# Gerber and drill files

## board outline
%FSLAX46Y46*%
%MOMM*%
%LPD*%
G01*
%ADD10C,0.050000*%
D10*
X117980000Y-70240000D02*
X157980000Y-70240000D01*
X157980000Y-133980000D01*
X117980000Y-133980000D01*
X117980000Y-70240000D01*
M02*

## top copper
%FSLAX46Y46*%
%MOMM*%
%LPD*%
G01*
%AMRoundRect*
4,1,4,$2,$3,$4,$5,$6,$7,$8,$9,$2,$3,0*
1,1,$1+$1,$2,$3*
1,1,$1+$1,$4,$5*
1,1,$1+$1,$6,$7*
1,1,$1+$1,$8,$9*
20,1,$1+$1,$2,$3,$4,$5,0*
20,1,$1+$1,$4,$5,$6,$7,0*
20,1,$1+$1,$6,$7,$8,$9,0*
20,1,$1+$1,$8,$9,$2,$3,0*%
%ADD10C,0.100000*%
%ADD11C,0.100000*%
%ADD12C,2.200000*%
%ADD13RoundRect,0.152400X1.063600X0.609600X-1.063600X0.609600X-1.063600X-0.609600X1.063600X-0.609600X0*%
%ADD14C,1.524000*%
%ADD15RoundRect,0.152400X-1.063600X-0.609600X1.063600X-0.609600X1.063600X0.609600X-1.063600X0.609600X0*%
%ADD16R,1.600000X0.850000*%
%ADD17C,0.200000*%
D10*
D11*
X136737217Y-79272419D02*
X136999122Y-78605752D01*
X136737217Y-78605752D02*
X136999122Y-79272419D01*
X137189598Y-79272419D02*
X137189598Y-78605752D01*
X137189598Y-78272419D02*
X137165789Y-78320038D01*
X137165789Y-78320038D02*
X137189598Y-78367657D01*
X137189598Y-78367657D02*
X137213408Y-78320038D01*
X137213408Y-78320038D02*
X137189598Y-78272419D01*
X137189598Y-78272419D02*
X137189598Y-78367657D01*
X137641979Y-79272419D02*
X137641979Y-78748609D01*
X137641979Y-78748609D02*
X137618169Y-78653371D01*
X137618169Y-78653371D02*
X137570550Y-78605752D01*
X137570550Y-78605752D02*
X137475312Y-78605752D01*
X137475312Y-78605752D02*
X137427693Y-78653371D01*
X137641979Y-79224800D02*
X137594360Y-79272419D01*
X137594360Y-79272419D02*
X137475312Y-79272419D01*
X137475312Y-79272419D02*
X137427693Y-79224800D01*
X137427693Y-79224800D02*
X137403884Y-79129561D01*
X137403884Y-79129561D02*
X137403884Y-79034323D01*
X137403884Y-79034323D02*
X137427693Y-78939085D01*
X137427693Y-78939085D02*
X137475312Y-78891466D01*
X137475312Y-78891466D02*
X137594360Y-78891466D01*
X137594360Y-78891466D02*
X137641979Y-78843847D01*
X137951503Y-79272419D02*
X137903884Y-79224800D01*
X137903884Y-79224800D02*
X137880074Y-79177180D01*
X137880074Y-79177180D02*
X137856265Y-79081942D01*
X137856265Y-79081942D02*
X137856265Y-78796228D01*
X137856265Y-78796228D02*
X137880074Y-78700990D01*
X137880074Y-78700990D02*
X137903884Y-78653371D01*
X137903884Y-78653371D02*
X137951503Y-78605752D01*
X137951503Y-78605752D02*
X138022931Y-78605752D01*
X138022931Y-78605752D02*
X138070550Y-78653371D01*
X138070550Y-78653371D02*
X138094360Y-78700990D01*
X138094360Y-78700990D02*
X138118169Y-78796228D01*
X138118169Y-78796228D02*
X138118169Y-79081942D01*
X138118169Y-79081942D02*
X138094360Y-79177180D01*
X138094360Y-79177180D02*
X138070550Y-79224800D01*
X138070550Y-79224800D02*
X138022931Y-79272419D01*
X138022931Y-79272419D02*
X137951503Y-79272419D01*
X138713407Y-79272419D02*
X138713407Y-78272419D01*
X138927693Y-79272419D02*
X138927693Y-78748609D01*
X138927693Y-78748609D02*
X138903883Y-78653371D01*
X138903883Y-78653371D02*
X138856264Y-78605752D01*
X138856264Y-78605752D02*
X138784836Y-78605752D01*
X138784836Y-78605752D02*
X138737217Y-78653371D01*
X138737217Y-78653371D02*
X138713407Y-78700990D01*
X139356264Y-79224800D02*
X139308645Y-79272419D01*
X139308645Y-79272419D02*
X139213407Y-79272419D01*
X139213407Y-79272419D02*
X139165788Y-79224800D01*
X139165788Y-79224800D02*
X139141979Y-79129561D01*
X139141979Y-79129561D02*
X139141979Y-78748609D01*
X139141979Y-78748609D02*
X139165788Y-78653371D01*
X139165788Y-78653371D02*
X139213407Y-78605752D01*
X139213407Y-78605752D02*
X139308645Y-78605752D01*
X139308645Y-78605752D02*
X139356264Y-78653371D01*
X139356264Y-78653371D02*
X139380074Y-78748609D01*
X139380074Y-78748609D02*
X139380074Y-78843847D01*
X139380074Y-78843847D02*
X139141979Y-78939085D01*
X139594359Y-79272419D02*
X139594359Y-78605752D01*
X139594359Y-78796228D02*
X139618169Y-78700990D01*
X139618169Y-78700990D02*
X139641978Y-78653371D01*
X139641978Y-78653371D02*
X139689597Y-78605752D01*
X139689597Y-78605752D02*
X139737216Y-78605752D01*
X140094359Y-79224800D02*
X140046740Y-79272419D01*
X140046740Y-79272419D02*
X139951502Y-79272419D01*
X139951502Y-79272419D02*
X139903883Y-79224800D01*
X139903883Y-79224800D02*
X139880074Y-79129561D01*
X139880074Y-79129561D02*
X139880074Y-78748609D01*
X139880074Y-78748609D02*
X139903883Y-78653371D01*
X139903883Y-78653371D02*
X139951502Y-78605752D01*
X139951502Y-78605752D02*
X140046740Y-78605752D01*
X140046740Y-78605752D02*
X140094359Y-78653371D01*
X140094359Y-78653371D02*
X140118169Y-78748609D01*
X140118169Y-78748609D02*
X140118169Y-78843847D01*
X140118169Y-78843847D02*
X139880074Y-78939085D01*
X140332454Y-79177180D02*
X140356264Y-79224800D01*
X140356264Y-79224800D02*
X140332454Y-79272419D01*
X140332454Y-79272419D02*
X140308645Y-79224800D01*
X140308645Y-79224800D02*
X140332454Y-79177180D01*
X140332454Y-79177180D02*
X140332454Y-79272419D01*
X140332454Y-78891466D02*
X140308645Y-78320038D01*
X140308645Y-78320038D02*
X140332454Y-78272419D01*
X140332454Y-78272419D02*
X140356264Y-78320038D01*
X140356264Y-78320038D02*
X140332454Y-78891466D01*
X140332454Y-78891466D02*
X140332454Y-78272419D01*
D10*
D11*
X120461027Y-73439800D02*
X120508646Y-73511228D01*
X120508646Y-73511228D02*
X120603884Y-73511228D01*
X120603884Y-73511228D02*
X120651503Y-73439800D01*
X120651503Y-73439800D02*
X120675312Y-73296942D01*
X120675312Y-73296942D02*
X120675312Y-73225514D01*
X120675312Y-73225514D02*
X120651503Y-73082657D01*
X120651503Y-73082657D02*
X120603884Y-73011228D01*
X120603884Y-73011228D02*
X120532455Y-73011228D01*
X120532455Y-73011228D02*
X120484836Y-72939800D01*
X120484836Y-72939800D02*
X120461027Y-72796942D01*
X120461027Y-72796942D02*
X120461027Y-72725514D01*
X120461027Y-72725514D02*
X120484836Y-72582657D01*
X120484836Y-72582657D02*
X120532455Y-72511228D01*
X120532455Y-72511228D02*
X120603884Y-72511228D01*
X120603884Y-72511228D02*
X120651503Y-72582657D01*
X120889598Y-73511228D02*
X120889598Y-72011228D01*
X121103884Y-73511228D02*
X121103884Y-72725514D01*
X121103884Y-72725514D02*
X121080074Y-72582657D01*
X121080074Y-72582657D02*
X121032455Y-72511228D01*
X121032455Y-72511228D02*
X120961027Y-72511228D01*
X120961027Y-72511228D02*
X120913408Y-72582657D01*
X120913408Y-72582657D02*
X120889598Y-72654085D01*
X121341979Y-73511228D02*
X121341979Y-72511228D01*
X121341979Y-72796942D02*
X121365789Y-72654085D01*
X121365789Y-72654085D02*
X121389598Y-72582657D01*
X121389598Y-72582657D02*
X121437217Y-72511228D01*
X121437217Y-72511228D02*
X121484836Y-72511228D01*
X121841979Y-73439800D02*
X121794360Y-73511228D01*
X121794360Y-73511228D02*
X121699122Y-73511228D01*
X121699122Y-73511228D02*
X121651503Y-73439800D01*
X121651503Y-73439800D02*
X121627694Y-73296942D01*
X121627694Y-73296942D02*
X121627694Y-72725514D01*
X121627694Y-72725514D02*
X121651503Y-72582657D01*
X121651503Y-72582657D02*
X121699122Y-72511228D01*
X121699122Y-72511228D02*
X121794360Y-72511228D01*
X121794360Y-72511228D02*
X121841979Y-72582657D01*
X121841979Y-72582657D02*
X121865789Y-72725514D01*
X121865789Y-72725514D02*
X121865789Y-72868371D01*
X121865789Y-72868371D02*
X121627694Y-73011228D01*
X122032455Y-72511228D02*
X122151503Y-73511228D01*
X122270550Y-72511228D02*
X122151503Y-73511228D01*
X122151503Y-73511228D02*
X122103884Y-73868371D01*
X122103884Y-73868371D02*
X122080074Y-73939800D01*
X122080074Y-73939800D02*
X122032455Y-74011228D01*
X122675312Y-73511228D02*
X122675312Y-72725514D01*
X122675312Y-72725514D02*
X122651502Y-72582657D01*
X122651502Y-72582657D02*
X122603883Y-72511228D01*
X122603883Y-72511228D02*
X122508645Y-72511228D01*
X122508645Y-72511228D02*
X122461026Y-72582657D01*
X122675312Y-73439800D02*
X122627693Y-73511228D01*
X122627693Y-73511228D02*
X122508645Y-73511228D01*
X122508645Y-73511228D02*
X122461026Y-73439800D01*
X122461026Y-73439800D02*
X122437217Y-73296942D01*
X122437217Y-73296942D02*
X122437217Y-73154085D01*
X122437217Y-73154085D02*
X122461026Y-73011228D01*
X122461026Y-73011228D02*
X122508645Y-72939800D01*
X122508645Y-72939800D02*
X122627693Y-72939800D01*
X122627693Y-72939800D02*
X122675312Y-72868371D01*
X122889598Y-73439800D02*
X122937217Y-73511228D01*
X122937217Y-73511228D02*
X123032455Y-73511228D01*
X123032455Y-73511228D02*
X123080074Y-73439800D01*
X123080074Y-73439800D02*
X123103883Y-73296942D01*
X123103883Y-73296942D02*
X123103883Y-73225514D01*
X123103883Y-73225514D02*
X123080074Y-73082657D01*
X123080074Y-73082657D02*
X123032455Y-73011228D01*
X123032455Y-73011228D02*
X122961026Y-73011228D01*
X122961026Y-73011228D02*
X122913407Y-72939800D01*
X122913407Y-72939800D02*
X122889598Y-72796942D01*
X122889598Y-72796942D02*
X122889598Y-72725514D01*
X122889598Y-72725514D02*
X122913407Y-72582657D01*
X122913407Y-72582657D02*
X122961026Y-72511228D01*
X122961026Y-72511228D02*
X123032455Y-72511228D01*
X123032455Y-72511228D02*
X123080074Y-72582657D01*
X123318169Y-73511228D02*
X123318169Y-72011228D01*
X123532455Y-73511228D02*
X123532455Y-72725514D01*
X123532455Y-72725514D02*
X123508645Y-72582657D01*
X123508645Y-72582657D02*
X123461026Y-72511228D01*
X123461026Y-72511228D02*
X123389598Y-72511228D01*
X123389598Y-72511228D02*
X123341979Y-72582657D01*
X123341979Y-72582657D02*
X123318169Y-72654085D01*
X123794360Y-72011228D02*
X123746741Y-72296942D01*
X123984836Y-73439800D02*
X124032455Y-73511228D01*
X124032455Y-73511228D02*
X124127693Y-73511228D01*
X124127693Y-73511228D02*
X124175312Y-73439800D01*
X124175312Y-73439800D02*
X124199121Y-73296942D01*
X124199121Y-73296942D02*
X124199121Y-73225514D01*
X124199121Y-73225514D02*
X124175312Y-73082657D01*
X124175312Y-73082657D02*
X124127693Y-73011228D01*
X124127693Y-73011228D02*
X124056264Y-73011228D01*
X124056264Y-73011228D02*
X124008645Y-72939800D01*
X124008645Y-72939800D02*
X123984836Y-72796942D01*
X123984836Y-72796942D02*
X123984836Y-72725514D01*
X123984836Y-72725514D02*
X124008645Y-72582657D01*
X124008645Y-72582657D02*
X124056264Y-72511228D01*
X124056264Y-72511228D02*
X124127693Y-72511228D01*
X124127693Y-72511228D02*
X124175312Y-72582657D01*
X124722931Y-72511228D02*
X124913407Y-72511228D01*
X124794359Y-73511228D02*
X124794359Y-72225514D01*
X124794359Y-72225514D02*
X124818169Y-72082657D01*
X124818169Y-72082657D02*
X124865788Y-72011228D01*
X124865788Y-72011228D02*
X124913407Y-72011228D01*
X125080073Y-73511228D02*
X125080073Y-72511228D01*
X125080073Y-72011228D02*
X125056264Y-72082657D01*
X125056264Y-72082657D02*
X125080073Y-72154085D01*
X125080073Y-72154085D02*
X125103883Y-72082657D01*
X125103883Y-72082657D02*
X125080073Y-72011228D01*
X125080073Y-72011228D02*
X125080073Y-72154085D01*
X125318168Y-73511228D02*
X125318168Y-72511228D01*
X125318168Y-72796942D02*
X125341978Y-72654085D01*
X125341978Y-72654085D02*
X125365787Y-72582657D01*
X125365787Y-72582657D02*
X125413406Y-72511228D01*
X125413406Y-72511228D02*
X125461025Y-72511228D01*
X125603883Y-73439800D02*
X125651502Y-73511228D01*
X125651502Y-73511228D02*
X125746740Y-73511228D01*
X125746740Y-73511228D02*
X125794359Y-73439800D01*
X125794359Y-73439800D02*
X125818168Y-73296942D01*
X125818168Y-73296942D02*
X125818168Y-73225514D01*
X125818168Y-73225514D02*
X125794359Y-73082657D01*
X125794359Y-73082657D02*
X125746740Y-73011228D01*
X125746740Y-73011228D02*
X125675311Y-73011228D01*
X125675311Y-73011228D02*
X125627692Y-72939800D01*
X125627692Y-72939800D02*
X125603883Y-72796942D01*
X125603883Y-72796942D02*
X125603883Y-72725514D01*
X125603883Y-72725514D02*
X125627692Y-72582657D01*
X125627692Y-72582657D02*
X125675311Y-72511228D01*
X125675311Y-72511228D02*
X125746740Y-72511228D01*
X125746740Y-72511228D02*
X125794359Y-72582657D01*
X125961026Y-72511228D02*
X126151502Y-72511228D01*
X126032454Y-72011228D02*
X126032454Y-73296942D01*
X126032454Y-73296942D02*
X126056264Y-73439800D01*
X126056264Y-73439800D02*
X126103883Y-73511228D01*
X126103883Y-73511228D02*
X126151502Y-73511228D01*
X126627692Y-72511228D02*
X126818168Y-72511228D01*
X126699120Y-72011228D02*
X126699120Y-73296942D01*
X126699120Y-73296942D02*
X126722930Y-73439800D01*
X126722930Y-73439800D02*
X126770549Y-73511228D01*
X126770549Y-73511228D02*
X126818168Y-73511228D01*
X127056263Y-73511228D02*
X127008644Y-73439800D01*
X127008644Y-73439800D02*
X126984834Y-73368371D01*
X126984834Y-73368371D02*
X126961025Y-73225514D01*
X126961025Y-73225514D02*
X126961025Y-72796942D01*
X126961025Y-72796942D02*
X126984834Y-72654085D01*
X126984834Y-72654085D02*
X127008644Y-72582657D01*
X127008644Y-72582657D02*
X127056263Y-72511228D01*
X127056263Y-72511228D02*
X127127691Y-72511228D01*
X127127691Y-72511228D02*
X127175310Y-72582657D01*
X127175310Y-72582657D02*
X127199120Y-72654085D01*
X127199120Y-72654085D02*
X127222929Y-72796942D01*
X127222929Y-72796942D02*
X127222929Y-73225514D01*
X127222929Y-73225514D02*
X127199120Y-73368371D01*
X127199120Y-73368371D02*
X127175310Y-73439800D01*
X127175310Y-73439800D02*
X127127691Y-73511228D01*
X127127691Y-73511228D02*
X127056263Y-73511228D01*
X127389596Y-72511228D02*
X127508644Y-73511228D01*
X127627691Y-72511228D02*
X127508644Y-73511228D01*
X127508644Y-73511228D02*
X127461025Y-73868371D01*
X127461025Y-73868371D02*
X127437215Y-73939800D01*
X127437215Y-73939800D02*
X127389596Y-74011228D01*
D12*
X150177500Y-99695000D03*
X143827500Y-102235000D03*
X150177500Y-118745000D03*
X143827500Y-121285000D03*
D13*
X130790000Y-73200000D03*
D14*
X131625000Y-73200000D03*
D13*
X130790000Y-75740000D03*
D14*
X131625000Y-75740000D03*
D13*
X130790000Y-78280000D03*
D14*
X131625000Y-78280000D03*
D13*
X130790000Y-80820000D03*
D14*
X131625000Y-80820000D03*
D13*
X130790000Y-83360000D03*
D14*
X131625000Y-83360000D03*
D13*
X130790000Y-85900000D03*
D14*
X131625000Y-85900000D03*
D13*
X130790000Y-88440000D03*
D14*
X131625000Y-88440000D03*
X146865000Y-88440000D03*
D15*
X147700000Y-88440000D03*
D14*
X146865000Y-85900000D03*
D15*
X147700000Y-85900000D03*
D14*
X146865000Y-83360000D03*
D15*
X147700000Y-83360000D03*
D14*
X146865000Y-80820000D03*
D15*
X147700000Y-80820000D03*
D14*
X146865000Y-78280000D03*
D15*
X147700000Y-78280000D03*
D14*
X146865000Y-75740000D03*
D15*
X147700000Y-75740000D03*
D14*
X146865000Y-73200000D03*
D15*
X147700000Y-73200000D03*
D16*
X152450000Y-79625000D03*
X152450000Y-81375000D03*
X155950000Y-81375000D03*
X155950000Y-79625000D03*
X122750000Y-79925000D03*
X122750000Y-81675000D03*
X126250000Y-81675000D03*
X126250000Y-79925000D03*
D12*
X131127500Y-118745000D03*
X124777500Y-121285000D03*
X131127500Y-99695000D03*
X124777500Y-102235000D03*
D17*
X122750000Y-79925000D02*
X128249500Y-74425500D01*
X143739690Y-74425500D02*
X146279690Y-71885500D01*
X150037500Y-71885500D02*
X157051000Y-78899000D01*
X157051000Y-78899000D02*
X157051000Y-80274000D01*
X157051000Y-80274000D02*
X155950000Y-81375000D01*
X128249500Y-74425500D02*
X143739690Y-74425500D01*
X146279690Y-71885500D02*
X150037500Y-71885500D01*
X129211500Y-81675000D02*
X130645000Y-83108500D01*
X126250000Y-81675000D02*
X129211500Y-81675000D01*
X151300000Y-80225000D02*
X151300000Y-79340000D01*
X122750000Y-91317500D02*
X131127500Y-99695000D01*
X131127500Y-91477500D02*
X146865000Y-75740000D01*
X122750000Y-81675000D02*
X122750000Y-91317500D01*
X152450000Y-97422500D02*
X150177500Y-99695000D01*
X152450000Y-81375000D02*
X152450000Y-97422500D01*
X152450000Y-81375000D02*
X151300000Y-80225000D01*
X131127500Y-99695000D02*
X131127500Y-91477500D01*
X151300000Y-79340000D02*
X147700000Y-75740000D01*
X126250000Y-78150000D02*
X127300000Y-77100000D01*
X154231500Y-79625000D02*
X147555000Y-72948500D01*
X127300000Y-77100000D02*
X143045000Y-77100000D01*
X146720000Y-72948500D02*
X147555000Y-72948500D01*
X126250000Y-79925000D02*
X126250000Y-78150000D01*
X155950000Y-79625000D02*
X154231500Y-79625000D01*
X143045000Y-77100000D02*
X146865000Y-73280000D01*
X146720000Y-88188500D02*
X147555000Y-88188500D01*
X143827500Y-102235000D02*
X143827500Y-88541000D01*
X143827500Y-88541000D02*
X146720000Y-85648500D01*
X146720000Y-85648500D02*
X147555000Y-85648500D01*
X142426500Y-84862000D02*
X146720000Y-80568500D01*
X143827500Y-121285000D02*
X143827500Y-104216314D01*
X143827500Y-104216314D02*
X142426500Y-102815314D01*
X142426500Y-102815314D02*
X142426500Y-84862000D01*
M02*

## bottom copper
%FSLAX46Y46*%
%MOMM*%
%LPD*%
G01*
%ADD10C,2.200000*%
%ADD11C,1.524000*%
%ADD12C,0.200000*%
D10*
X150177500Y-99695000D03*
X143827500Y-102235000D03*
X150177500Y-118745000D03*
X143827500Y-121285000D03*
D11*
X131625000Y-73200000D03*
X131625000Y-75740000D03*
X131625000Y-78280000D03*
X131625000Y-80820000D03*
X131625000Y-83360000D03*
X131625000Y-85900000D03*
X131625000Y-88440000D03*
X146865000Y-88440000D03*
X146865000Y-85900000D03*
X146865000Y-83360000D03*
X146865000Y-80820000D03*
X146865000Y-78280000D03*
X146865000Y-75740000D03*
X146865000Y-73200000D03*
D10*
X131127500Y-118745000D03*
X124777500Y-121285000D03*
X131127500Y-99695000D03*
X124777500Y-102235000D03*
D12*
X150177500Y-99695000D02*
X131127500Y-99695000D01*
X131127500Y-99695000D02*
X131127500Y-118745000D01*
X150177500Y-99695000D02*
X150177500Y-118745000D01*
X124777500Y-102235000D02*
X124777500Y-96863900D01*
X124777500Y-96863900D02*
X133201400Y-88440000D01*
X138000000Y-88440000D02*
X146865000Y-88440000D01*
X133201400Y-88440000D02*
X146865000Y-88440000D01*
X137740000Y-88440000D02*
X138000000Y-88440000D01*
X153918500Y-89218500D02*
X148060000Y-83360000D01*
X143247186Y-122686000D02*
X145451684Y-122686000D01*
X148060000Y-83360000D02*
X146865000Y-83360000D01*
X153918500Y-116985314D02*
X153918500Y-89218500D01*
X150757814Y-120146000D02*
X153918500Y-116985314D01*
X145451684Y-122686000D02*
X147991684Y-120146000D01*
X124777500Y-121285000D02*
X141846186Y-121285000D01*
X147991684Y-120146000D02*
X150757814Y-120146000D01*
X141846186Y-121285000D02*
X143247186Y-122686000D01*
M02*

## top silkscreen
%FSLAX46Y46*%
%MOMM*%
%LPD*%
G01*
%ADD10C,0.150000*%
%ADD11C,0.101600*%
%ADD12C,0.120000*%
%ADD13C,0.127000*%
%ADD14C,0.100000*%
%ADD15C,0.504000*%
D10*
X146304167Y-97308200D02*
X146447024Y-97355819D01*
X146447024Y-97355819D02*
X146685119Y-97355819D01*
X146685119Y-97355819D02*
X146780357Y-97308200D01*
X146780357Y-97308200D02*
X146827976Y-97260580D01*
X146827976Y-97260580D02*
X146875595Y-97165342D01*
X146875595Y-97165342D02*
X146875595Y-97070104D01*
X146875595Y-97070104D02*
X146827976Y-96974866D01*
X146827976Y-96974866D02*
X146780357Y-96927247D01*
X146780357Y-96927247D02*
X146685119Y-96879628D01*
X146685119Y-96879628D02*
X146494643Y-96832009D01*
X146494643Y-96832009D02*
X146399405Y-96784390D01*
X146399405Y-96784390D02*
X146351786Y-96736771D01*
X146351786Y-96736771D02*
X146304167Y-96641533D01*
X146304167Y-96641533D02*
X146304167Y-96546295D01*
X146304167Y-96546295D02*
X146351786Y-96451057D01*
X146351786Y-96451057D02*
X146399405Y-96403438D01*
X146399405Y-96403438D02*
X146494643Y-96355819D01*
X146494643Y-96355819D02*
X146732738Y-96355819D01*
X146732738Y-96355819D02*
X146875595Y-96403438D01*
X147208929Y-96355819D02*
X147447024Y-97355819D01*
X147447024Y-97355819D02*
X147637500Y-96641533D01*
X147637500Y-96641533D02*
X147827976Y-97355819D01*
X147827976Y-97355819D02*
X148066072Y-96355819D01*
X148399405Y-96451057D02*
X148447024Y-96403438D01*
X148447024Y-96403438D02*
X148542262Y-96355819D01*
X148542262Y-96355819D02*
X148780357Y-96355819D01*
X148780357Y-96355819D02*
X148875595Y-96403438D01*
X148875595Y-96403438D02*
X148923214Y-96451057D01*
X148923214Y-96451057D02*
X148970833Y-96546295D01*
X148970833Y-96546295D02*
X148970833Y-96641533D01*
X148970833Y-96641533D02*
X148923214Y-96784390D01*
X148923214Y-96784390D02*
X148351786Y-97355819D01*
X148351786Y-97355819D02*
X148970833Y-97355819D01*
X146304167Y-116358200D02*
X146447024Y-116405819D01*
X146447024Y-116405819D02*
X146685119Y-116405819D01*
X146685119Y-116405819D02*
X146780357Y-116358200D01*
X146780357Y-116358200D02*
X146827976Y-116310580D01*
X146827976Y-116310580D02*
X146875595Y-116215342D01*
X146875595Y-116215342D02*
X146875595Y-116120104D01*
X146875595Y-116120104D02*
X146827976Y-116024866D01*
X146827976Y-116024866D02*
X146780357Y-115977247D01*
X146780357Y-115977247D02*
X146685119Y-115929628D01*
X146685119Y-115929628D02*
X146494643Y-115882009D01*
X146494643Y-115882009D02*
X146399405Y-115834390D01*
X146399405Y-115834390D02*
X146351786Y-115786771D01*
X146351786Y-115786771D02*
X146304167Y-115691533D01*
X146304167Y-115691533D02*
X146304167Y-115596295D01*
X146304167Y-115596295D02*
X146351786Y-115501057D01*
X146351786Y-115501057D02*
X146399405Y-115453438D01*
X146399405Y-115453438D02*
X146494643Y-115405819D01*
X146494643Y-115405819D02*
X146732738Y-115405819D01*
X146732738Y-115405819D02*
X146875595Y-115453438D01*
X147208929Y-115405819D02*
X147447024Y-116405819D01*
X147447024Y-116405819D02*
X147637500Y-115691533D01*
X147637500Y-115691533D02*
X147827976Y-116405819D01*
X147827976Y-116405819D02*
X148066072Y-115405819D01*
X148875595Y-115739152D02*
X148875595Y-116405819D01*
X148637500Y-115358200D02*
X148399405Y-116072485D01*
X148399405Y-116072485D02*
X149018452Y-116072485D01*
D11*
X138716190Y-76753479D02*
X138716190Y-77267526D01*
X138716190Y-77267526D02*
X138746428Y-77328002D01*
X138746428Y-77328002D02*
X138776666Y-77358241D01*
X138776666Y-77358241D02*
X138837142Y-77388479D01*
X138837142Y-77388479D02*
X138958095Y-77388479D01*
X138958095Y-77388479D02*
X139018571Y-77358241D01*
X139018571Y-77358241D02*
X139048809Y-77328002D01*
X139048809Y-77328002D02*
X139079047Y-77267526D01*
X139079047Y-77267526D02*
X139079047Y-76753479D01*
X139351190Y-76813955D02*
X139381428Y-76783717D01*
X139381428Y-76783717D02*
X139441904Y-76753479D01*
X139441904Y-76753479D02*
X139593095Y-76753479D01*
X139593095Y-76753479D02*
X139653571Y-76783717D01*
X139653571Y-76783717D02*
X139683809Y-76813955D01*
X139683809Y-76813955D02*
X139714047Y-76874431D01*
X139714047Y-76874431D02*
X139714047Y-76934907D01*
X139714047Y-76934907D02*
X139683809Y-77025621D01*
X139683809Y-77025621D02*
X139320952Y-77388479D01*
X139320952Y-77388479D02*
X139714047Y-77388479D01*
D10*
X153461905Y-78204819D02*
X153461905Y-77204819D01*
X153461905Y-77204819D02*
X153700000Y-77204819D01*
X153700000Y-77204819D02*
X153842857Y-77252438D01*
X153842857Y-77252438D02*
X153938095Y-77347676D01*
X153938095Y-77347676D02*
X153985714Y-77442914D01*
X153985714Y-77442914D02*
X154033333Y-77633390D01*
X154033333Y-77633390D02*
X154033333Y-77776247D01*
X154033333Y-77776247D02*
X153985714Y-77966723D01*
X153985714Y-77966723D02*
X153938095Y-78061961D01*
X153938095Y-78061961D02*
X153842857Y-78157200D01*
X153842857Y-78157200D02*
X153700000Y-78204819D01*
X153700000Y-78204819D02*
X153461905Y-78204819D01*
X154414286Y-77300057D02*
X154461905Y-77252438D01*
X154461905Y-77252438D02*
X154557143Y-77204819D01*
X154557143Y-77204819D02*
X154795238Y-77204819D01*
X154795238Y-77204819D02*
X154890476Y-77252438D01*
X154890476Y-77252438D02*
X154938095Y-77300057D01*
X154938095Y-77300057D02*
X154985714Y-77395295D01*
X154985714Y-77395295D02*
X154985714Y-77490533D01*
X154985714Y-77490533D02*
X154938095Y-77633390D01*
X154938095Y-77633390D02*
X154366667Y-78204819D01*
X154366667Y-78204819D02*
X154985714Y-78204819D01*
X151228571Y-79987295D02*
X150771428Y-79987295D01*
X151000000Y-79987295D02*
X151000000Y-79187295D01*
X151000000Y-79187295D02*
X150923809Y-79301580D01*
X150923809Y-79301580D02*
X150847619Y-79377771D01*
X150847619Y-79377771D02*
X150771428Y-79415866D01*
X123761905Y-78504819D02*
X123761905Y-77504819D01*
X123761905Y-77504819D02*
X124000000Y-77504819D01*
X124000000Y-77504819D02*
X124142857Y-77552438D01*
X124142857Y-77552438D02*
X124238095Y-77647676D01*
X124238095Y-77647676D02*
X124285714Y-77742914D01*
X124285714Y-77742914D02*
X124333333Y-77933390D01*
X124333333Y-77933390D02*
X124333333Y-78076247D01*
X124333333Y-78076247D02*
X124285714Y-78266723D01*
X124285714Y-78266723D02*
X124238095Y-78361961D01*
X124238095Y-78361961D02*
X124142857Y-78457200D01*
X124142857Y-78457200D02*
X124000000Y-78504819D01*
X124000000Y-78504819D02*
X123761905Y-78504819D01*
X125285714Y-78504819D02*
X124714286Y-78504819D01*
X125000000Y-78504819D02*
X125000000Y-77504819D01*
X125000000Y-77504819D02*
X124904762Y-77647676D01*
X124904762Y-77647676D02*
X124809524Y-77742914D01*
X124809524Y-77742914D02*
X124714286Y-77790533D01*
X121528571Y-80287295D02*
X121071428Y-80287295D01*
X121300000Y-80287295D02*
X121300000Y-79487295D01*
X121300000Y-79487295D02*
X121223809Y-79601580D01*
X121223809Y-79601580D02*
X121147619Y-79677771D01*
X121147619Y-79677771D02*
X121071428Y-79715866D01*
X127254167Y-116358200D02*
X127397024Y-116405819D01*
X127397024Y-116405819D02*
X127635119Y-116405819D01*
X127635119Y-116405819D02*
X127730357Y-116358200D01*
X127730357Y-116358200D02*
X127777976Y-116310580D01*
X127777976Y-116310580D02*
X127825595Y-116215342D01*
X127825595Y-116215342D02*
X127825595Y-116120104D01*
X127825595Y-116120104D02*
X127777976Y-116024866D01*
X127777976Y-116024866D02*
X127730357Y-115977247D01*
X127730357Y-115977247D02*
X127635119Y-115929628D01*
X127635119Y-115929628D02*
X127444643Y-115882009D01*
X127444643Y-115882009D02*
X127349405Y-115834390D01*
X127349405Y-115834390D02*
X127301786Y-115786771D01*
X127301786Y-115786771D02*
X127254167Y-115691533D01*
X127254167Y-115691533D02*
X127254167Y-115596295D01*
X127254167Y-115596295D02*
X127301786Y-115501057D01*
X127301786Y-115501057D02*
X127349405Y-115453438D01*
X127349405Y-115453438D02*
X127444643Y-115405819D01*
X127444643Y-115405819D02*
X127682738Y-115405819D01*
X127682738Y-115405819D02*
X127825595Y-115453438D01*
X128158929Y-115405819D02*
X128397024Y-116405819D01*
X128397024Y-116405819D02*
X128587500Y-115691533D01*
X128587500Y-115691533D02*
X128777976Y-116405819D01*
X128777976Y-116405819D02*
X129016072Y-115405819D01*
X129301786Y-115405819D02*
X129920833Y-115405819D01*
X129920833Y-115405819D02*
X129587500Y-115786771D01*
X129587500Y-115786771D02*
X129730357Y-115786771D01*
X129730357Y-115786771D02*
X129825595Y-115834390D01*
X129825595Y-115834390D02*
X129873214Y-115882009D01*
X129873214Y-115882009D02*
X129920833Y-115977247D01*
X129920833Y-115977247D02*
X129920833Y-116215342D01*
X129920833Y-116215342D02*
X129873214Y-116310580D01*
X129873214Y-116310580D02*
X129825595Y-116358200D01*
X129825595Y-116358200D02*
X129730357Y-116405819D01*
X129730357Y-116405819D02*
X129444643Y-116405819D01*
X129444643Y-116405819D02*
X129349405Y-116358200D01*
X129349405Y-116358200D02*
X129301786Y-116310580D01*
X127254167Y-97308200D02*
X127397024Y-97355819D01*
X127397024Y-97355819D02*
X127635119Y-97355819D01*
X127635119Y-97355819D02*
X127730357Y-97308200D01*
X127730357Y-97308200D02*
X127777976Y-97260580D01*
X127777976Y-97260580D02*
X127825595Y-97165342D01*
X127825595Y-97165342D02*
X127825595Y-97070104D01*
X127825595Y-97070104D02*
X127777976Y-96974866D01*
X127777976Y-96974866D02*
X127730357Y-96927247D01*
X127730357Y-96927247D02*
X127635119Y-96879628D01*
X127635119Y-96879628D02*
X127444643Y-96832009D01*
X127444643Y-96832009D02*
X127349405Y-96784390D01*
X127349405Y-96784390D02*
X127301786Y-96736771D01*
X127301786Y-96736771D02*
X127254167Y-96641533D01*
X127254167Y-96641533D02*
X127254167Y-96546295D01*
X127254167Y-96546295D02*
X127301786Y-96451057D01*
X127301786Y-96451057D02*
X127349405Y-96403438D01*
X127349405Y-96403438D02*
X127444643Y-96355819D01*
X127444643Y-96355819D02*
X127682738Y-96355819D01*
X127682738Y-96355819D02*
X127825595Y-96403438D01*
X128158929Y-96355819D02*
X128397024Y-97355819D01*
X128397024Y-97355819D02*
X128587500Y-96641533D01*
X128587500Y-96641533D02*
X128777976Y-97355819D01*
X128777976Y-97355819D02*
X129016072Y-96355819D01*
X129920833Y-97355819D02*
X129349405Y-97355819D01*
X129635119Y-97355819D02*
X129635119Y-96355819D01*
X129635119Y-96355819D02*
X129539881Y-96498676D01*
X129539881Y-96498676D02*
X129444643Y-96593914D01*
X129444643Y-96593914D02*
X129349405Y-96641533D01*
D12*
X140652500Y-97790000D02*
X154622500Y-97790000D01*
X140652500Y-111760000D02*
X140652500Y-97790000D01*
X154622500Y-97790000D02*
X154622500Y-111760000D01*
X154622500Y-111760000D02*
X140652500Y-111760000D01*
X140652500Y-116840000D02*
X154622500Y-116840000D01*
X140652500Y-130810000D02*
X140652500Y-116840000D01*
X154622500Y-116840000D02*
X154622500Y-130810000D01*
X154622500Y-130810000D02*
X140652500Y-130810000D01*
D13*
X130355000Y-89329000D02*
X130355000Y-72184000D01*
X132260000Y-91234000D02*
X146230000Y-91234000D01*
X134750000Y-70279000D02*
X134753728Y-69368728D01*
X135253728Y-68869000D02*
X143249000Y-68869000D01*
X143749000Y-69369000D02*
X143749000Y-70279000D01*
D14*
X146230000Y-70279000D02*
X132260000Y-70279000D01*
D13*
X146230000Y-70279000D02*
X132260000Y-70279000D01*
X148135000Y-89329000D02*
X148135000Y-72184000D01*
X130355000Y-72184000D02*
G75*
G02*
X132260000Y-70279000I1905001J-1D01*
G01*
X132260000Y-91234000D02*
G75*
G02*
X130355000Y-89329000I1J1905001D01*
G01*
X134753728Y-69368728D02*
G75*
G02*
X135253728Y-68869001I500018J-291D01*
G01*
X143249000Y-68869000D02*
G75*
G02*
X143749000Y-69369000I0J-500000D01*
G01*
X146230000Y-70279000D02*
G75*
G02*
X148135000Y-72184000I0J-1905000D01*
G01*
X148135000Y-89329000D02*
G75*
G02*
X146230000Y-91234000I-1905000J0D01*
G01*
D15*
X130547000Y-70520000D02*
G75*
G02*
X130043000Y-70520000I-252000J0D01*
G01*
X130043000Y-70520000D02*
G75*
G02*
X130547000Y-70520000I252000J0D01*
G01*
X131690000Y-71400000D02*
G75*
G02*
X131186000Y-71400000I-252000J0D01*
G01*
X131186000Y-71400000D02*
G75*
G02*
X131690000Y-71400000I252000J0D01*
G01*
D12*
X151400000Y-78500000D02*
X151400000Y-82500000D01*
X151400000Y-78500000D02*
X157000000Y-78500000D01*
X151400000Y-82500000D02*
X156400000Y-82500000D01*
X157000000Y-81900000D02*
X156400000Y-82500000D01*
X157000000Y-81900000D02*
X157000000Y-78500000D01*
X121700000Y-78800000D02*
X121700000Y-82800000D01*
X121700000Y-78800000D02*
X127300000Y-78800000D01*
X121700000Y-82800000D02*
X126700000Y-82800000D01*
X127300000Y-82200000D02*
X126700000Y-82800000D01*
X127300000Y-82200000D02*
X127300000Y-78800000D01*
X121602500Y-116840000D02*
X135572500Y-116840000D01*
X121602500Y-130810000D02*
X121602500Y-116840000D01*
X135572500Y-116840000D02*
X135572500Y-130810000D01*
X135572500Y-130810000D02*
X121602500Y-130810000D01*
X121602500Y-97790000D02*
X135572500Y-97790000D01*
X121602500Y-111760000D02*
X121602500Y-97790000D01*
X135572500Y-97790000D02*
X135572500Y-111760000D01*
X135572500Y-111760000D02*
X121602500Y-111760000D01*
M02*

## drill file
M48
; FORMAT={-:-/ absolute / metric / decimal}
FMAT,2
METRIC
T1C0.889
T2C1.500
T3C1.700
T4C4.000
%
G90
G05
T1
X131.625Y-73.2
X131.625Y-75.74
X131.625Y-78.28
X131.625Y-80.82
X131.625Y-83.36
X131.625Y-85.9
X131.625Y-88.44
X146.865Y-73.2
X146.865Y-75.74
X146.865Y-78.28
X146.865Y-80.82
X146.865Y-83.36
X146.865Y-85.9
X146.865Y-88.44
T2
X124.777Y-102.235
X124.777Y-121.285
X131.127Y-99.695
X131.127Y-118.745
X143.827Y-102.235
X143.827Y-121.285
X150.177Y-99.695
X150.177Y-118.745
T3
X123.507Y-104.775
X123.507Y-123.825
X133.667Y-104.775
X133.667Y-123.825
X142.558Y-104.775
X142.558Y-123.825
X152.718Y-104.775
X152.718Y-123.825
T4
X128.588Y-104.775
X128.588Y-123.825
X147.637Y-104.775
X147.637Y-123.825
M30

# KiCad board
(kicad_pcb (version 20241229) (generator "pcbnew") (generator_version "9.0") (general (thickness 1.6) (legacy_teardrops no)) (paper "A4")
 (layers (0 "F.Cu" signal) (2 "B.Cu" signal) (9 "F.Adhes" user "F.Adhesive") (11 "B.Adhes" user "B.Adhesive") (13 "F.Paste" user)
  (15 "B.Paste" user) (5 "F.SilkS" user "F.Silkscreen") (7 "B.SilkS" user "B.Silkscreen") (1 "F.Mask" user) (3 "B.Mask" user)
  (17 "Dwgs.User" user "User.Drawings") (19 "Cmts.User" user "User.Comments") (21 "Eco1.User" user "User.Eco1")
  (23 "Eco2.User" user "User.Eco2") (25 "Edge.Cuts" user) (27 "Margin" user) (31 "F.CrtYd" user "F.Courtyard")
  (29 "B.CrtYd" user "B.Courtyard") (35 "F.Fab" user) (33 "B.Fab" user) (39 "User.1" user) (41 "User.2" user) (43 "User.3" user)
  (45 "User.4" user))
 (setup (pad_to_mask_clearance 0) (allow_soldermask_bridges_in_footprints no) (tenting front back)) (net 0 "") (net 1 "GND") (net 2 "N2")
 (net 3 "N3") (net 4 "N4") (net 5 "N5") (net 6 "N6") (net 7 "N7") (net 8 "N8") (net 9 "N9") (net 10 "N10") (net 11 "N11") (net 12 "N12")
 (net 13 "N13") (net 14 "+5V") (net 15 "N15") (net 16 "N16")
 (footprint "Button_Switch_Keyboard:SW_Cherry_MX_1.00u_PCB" (layer "F.Cu") (at 150.1775 99.695)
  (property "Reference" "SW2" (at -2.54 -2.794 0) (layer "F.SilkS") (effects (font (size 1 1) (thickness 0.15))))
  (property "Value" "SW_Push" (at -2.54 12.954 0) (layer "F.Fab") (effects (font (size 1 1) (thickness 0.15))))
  (fp_line (start -9.525 -1.905) (end 4.445 -1.905) (stroke (width 0.12) (type solid)) (layer "F.SilkS"))
  (fp_line (start -9.525 12.065) (end -9.525 -1.905) (stroke (width 0.12) (type solid)) (layer "F.SilkS"))
  (fp_line (start 4.445 -1.905) (end 4.445 12.065) (stroke (width 0.12) (type solid)) (layer "F.SilkS"))
  (fp_line (start 4.445 12.065) (end -9.525 12.065) (stroke (width 0.12) (type solid)) (layer "F.SilkS"))
  (pad "" np_thru_hole circle (at -7.62 5.08) (size 1.7 1.7) (drill 1.7) (layers "*.Cu" "*.Mask"))
  (pad "" np_thru_hole circle (at -2.54 5.08) (size 4 4) (drill 4) (layers "*.Cu" "*.Mask"))
  (pad "" np_thru_hole circle (at 2.54 5.08) (size 1.7 1.7) (drill 1.7) (layers "*.Cu" "*.Mask"))
  (pad "1" thru_hole circle (at 0 0) (size 2.2 2.2) (drill 1.5) (layers "*.Cu" "*.Mask") (remove_unused_layers no) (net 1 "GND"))
  (pad "2" thru_hole circle (at -6.35 2.54) (size 2.2 2.2) (drill 1.5) (layers "*.Cu" "*.Mask") (remove_unused_layers no) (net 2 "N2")))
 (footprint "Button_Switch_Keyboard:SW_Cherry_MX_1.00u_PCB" (layer "F.Cu") (at 150.1775 118.745)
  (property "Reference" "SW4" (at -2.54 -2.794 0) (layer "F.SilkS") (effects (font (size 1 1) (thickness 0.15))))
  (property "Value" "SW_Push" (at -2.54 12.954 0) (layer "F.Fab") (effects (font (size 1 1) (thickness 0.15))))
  (fp_line (start -9.525 -1.905) (end 4.445 -1.905) (stroke (width 0.12) (type solid)) (layer "F.SilkS"))
  (fp_line (start -9.525 12.065) (end -9.525 -1.905) (stroke (width 0.12) (type solid)) (layer "F.SilkS"))
  (fp_line (start 4.445 -1.905) (end 4.445 12.065) (stroke (width 0.12) (type solid)) (layer "F.SilkS"))
  (fp_line (start 4.445 12.065) (end -9.525 12.065) (stroke (width 0.12) (type solid)) (layer "F.SilkS"))
  (pad "" np_thru_hole circle (at -7.62 5.08) (size 1.7 1.7) (drill 1.7) (layers "*.Cu" "*.Mask"))
  (pad "" np_thru_hole circle (at -2.54 5.08) (size 4 4) (drill 4) (layers "*.Cu" "*.Mask"))
  (pad "" np_thru_hole circle (at 2.54 5.08) (size 1.7 1.7) (drill 1.7) (layers "*.Cu" "*.Mask"))
  (pad "1" thru_hole circle (at 0 0) (size 2.2 2.2) (drill 1.5) (layers "*.Cu" "*.Mask") (remove_unused_layers no) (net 1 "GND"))
  (pad "2" thru_hole circle (at -6.35 2.54) (size 2.2 2.2) (drill 1.5) (layers "*.Cu" "*.Mask") (remove_unused_layers no) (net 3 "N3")))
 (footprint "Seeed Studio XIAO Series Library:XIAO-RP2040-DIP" (layer "F.Cu") (at 139.245 80.82)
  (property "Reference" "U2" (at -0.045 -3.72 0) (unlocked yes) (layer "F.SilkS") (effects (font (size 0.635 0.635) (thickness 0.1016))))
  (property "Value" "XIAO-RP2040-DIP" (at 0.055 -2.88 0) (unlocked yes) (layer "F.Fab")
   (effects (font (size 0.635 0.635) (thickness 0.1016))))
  (fp_line (start -8.89 8.509) (end -8.89 -8.636) (stroke (width 0.127) (type solid)) (layer "F.SilkS"))
  (fp_line (start -6.985 10.414) (end 6.985 10.414) (stroke (width 0.127) (type solid)) (layer "F.SilkS"))
  (fp_line (start -4.495 -10.541) (end -4.491272 -11.451272) (stroke (width 0.127) (type solid)) (layer "F.SilkS"))
  (fp_line (start -3.991272 -11.951) (end 4.004 -11.951) (stroke (width 0.127) (type solid)) (layer "F.SilkS"))
  (fp_line (start 4.504 -11.451) (end 4.504 -10.541) (stroke (width 0.127) (type solid)) (layer "F.SilkS"))
  (fp_line (start 6.985 -10.541) (end -6.985 -10.541) (stroke (width 0.1) (type solid)) (layer "F.SilkS"))
  (fp_line (start 6.985 -10.541) (end -6.985 -10.541) (stroke (width 0.127) (type solid)) (layer "F.SilkS"))
  (fp_line (start 8.89 8.509) (end 8.89 -8.636) (stroke (width 0.127) (type solid)) (layer "F.SilkS"))
  (fp_arc (start -8.89 -8.636) (mid -8.332038 -9.983038) (end -6.985 -10.541) (stroke (width 0.127) (type solid)) (layer "F.SilkS"))
  (fp_arc (start -6.985 10.414) (mid -8.332038 9.856038) (end -8.89 8.509) (stroke (width 0.127) (type solid)) (layer "F.SilkS"))
  (fp_arc (start -4.491272 -11.451272) (mid -4.344728 -11.80464) (end -3.991272 -11.951) (stroke (width 0.127) (type default))
   (layer "F.SilkS"))
  (fp_arc (start 4.004 -11.951) (mid 4.357553 -11.804553) (end 4.504 -11.451) (stroke (width 0.127) (type default)) (layer "F.SilkS"))
  (fp_arc (start 6.985 -10.541) (mid 8.332038 -9.983038) (end 8.89 -8.636) (stroke (width 0.127) (type solid)) (layer "F.SilkS"))
  (fp_arc (start 8.89 8.509) (mid 8.332038 9.856038) (end 6.985 10.414) (stroke (width 0.127) (type solid)) (layer "F.SilkS"))
  (fp_circle (center -8.95 -10.3) (end -8.95 -10.554) (stroke (width 0.5) (type solid)) (fill yes) (layer "F.SilkS"))
  (fp_circle (center -7.807 -9.42) (end -7.807 -9.674) (stroke (width 0.5) (type solid)) (fill yes) (layer "F.SilkS"))
  (pad "1" smd roundrect (at -8.455 -7.62 180) (size 2.432 1.524) (layers "F.Cu" "F.Mask") (roundrect_rratio 0.1) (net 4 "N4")
   (thermal_bridge_angle 45))
  (pad "1" thru_hole circle (at -7.62 -7.62 180) (size 1.524 1.524) (drill 0.889) (layers "*.Cu" "*.Mask") (remove_unused_layers no)
   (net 4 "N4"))
  (pad "2" smd roundrect (at -8.455 -5.08 180) (size 2.432 1.524) (layers "F.Cu" "F.Mask") (roundrect_rratio 0.1) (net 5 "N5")
   (thermal_bridge_angle 45))
  (pad "2" thru_hole circle (at -7.62 -5.08 180) (size 1.524 1.524) (drill 0.889) (layers "*.Cu" "*.Mask") (remove_unused_layers no)
   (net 5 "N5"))
  (pad "3" smd roundrect (at -8.455 -2.54 180) (size 2.432 1.524) (layers "F.Cu" "F.Mask") (roundrect_rratio 0.1) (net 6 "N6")
   (thermal_bridge_angle 45))
  (pad "3" thru_hole circle (at -7.62 -2.54 180) (size 1.524 1.524) (drill 0.889) (layers "*.Cu" "*.Mask") (remove_unused_layers no)
   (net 6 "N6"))
  (pad "4" smd roundrect (at -8.455 0 180) (size 2.432 1.524) (layers "F.Cu" "F.Mask") (roundrect_rratio 0.1) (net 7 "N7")
   (thermal_bridge_angle 45))
  (pad "4" thru_hole circle (at -7.62 0 180) (size 1.524 1.524) (drill 0.889) (layers "*.Cu" "*.Mask") (remove_unused_layers no)
   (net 7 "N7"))
  (pad "5" smd roundrect (at -8.455 2.54 180) (size 2.432 1.524) (layers "F.Cu" "F.Mask") (roundrect_rratio 0.1) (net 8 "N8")
   (thermal_bridge_angle 45))
  (pad "5" thru_hole circle (at -7.62 2.54 180) (size 1.524 1.524) (drill 0.889) (layers "*.Cu" "*.Mask") (remove_unused_layers no)
   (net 8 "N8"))
  (pad "6" smd roundrect (at -8.455 5.08 180) (size 2.432 1.524) (layers "F.Cu" "F.Mask") (roundrect_rratio 0.1) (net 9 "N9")
   (thermal_bridge_angle 45))
  (pad "6" thru_hole circle (at -7.62 5.08 180) (size 1.524 1.524) (drill 0.889) (layers "*.Cu" "*.Mask") (remove_unused_layers no)
   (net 9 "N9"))
  (pad "7" smd roundrect (at -8.455 7.62 180) (size 2.432 1.524) (layers "F.Cu" "F.Mask") (roundrect_rratio 0.1) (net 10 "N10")
   (thermal_bridge_angle 45))
  (pad "7" thru_hole circle (at -7.62 7.62 180) (size 1.524 1.524) (drill 0.889) (layers "*.Cu" "*.Mask") (remove_unused_layers no)
   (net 10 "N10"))
  (pad "8" thru_hole circle (at 7.62 7.62) (size 1.524 1.524) (drill 0.889) (layers "*.Cu" "*.Mask") (remove_unused_layers no)
   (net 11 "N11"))
  (pad "8" smd roundrect (at 8.455 7.62) (size 2.432 1.524) (layers "F.Cu" "F.Mask") (roundrect_rratio 0.1) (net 11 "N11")
   (thermal_bridge_angle 45))
  (pad "9" thru_hole circle (at 7.62 5.08) (size 1.524 1.524) (drill 0.889) (layers "*.Cu" "*.Mask") (remove_unused_layers no) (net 2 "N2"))
  (pad "9" smd roundrect (at 8.455 5.08) (size 2.432 1.524) (layers "F.Cu" "F.Mask") (roundrect_rratio 0.1) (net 2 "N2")
   (thermal_bridge_angle 45))
  (pad "10" thru_hole circle (at 7.62 2.54) (size 1.524 1.524) (drill 0.889) (layers "*.Cu" "*.Mask") (remove_unused_layers no)
   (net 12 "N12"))
  (pad "10" smd roundrect (at 8.455 2.54) (size 2.432 1.524) (layers "F.Cu" "F.Mask") (roundrect_rratio 0.1) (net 12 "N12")
   (thermal_bridge_angle 45))
  (pad "11" thru_hole circle (at 7.62 0) (size 1.524 1.524) (drill 0.889) (layers "*.Cu" "*.Mask") (remove_unused_layers no) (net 3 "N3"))
  (pad "11" smd roundrect (at 8.455 0) (size 2.432 1.524) (layers "F.Cu" "F.Mask") (roundrect_rratio 0.1) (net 3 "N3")
   (thermal_bridge_angle 45))
  (pad "12" thru_hole circle (at 7.62 -2.54) (size 1.524 1.524) (drill 0.889) (layers "*.Cu" "*.Mask") (remove_unused_layers no)
   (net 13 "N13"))
  (pad "12" smd roundrect (at 8.455 -2.54) (size 2.432 1.524) (layers "F.Cu" "F.Mask") (roundrect_rratio 0.1) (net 13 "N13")
   (thermal_bridge_angle 45))
  (pad "13" thru_hole circle (at 7.62 -5.08) (size 1.524 1.524) (drill 0.889) (layers "*.Cu" "*.Mask") (remove_unused_layers no)
   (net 1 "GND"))
  (pad "13" smd roundrect (at 8.455 -5.08) (size 2.432 1.524) (layers "F.Cu" "F.Mask") (roundrect_rratio 0.1) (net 1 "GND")
   (thermal_bridge_angle 45))
  (pad "14" thru_hole circle (at 7.62 -7.62) (size 1.524 1.524) (drill 0.889) (layers "*.Cu" "*.Mask") (remove_unused_layers no)
   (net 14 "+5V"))
  (pad "14" smd roundrect (at 8.455 -7.62) (size 2.432 1.524) (layers "F.Cu" "F.Mask") (roundrect_rratio 0.1) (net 14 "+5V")
   (thermal_bridge_angle 45)))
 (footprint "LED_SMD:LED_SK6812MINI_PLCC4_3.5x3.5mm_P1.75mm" (layer "F.Cu") (at 154.2 80.5)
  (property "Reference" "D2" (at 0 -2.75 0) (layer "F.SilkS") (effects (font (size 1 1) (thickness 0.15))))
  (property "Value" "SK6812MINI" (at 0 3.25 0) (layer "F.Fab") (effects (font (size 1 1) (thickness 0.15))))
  (fp_line (start -2.8 -2) (end -2.8 2) (stroke (width 0.12) (type default)) (layer "F.SilkS"))
  (fp_line (start -2.8 -2) (end 2.8 -2) (stroke (width 0.12) (type solid)) (layer "F.SilkS"))
  (fp_line (start -2.8 2) (end 2.2 2) (stroke (width 0.12) (type solid)) (layer "F.SilkS"))
  (fp_line (start 2.8 1.4) (end 2.2 2) (stroke (width 0.12) (type default)) (layer "F.SilkS"))
  (fp_line (start 2.8 1.4) (end 2.8 -2) (stroke (width 0.12) (type solid)) (layer "F.SilkS"))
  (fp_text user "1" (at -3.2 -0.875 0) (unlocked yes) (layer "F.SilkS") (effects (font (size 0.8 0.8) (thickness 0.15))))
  (pad "1" smd rect (at -1.75 -0.875) (size 1.6 0.85) (layers "F.Cu" "F.Mask" "F.Paste") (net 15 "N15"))
  (pad "2" smd rect (at -1.75 0.875) (size 1.6 0.85) (layers "F.Cu" "F.Mask" "F.Paste") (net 1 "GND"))
  (pad "3" smd rect (at 1.75 0.875) (size 1.6 0.85) (layers "F.Cu" "F.Mask" "F.Paste") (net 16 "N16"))
  (pad "4" smd rect (at 1.75 -0.875) (size 1.6 0.85) (layers "F.Cu" "F.Mask" "F.Paste") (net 14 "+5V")))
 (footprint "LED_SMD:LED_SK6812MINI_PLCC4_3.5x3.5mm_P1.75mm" (layer "F.Cu") (at 124.5 80.8)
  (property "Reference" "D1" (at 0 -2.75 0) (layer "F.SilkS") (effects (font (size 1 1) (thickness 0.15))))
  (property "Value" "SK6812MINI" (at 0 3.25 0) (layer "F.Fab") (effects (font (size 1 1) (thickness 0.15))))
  (fp_line (start -2.8 -2) (end -2.8 2) (stroke (width 0.12) (type default)) (layer "F.SilkS"))
  (fp_line (start -2.8 -2) (end 2.8 -2) (stroke (width 0.12) (type solid)) (layer "F.SilkS"))
  (fp_line (start -2.8 2) (end 2.2 2) (stroke (width 0.12) (type solid)) (layer "F.SilkS"))
  (fp_line (start 2.8 1.4) (end 2.2 2) (stroke (width 0.12) (type default)) (layer "F.SilkS"))
  (fp_line (start 2.8 1.4) (end 2.8 -2) (stroke (width 0.12) (type solid)) (layer "F.SilkS"))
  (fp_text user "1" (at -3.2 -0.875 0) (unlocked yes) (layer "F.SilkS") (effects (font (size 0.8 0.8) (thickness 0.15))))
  (pad "1" smd rect (at -1.75 -0.875) (size 1.6 0.85) (layers "F.Cu" "F.Mask" "F.Paste") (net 16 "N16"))
  (pad "2" smd rect (at -1.75 0.875) (size 1.6 0.85) (layers "F.Cu" "F.Mask" "F.Paste") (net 1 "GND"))
  (pad "3" smd rect (at 1.75 0.875) (size 1.6 0.85) (layers "F.Cu" "F.Mask" "F.Paste") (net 8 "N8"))
  (pad "4" smd rect (at 1.75 -0.875) (size 1.6 0.85) (layers "F.Cu" "F.Mask" "F.Paste") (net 14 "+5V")))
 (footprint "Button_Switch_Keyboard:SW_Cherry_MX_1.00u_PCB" (layer "F.Cu") (at 131.1275 118.745)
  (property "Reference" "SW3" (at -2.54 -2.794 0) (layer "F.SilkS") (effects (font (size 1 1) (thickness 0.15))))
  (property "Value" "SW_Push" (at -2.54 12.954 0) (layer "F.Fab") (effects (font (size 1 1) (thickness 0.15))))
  (fp_line (start -9.525 -1.905) (end 4.445 -1.905) (stroke (width 0.12) (type solid)) (layer "F.SilkS"))
  (fp_line (start -9.525 12.065) (end -9.525 -1.905) (stroke (width 0.12) (type solid)) (layer "F.SilkS"))
  (fp_line (start 4.445 -1.905) (end 4.445 12.065) (stroke (width 0.12) (type solid)) (layer "F.SilkS"))
  (fp_line (start 4.445 12.065) (end -9.525 12.065) (stroke (width 0.12) (type solid)) (layer "F.SilkS"))
  (pad "" np_thru_hole circle (at -7.62 5.08) (size 1.7 1.7) (drill 1.7) (layers "*.Cu" "*.Mask"))
  (pad "" np_thru_hole circle (at -2.54 5.08) (size 4 4) (drill 4) (layers "*.Cu" "*.Mask"))
  (pad "" np_thru_hole circle (at 2.54 5.08) (size 1.7 1.7) (drill 1.7) (layers "*.Cu" "*.Mask"))
  (pad "1" thru_hole circle (at 0 0) (size 2.2 2.2) (drill 1.5) (layers "*.Cu" "*.Mask") (remove_unused_layers no) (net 1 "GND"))
  (pad "2" thru_hole circle (at -6.35 2.54) (size 2.2 2.2) (drill 1.5) (layers "*.Cu" "*.Mask") (remove_unused_layers no) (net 12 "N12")))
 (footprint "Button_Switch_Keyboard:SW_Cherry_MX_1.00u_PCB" (layer "F.Cu") (at 131.1275 99.695)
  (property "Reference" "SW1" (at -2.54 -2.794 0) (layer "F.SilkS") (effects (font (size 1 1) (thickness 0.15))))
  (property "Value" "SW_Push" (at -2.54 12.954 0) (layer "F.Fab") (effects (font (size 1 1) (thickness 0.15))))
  (fp_line (start -9.525 -1.905) (end 4.445 -1.905) (stroke (width 0.12) (type solid)) (layer "F.SilkS"))
  (fp_line (start -9.525 12.065) (end -9.525 -1.905) (stroke (width 0.12) (type solid)) (layer "F.SilkS"))
  (fp_line (start 4.445 -1.905) (end 4.445 12.065) (stroke (width 0.12) (type solid)) (layer "F.SilkS"))
  (fp_line (start 4.445 12.065) (end -9.525 12.065) (stroke (width 0.12) (type solid)) (layer "F.SilkS"))
  (pad "" np_thru_hole circle (at -7.62 5.08) (size 1.7 1.7) (drill 1.7) (layers "*.Cu" "*.Mask"))
  (pad "" np_thru_hole circle (at -2.54 5.08) (size 4 4) (drill 4) (layers "*.Cu" "*.Mask"))
  (pad "" np_thru_hole circle (at 2.54 5.08) (size 1.7 1.7) (drill 1.7) (layers "*.Cu" "*.Mask"))
  (pad "1" thru_hole circle (at 0 0) (size 2.2 2.2) (drill 1.5) (layers "*.Cu" "*.Mask") (remove_unused_layers no) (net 1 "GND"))
  (pad "2" thru_hole circle (at -6.35 2.54) (size 2.2 2.2) (drill 1.5) (layers "*.Cu" "*.Mask") (remove_unused_layers no) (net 11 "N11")))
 (gr_rect (start 117.98 70.24) (end 157.98 133.98) (stroke (width 0.05) (type default)) (fill no) (layer "Edge.Cuts"))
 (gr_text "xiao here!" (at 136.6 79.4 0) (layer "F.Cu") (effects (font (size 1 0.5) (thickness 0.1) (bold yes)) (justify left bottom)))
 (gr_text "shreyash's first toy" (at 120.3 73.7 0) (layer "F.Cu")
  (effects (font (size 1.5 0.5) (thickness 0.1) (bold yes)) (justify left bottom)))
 (segment (start 122.75 79.925) (end 128.2495 74.4255) (width 0.2) (layer "F.Cu") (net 16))
 (segment (start 143.73969 74.4255) (end 146.27969 71.8855) (width 0.2) (layer "F.Cu") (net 16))
 (segment (start 150.0375 71.8855) (end 157.051 78.899) (width 0.2) (layer "F.Cu") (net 16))
 (segment (start 157.051 78.899) (end 157.051 80.274) (width 0.2) (layer "F.Cu") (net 16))
 (segment (start 157.051 80.274) (end 155.95 81.375) (width 0.2) (layer "F.Cu") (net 16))
 (segment (start 128.2495 74.4255) (end 143.73969 74.4255) (width 0.2) (layer "F.Cu") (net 16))
 (segment (start 146.27969 71.8855) (end 150.0375 71.8855) (width 0.2) (layer "F.Cu") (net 16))
 (segment (start 129.2115 81.675) (end 130.645 83.1085) (width 0.2) (layer "F.Cu") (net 8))
 (segment (start 126.25 81.675) (end 129.2115 81.675) (width 0.2) (layer "F.Cu") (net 8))
 (segment (start 151.3 80.225) (end 151.3 79.34) (width 0.2) (layer "F.Cu") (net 1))
 (segment (start 122.75 91.3175) (end 131.1275 99.695) (width 0.2) (layer "F.Cu") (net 1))
 (segment (start 131.1275 91.4775) (end 146.865 75.74) (width 0.2) (layer "F.Cu") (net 1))
 (segment (start 122.75 81.675) (end 122.75 91.3175) (width 0.2) (layer "F.Cu") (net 1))
 (segment (start 152.45 97.4225) (end 150.1775 99.695) (width 0.2) (layer "F.Cu") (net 1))
 (segment (start 152.45 81.375) (end 152.45 97.4225) (width 0.2) (layer "F.Cu") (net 1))
 (segment (start 152.45 81.375) (end 151.3 80.225) (width 0.2) (layer "F.Cu") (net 1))
 (segment (start 131.1275 99.695) (end 131.1275 91.4775) (width 0.2) (layer "F.Cu") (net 1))
 (segment (start 151.3 79.34) (end 147.7 75.74) (width 0.2) (layer "F.Cu") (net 1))
 (segment (start 150.1775 99.695) (end 131.1275 99.695) (width 0.2) (layer "B.Cu") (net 1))
 (segment (start 131.1275 99.695) (end 131.1275 118.745) (width 0.2) (layer "B.Cu") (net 1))
 (segment (start 150.1775 99.695) (end 150.1775 118.745) (width 0.2) (layer "B.Cu") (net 1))
 (segment (start 126.25 78.15) (end 127.3 77.1) (width 0.2) (layer "F.Cu") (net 14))
 (segment (start 154.2315 79.625) (end 147.555 72.9485) (width 0.2) (layer "F.Cu") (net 14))
 (segment (start 127.3 77.1) (end 143.045 77.1) (width 0.2) (layer "F.Cu") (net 14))
 (segment (start 146.72 72.9485) (end 147.555 72.9485) (width 0.2) (layer "F.Cu") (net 14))
 (segment (start 126.25 79.925) (end 126.25 78.15) (width 0.2) (layer "F.Cu") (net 14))
 (segment (start 155.95 79.625) (end 154.2315 79.625) (width 0.2) (layer "F.Cu") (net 14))
 (segment (start 143.045 77.1) (end 146.865 73.28) (width 0.2) (layer "F.Cu") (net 14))
 (segment (start 146.72 88.1885) (end 147.555 88.1885) (width 0.2) (layer "F.Cu") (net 11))
 (segment (start 124.7775 102.235) (end 124.7775 96.8639) (width 0.2) (layer "B.Cu") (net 11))
 (segment (start 124.7775 96.8639) (end 133.2014 88.44) (width 0.2) (layer "B.Cu") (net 11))
 (segment (start 138 88.44) (end 146.865 88.44) (width 0.2) (layer "B.Cu") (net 11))
 (segment (start 133.2014 88.44) (end 146.865 88.44) (width 0.2) (layer "B.Cu") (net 11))
 (segment (start 137.74 88.44) (end 138 88.44) (width 0.2) (layer "B.Cu") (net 11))
 (segment (start 143.8275 102.235) (end 143.8275 88.541) (width 0.2) (layer "F.Cu") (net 2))
 (segment (start 143.8275 88.541) (end 146.72 85.6485) (width 0.2) (layer "F.Cu") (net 2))
 (segment (start 146.72 85.6485) (end 147.555 85.6485) (width 0.2) (layer "F.Cu") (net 2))
 (segment (start 153.9185 89.2185) (end 148.06 83.36) (width 0.2) (layer "B.Cu") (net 12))
 (segment (start 143.247186 122.686) (end 145.451684 122.686) (width 0.2) (layer "B.Cu") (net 12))
 (segment (start 148.06 83.36) (end 146.865 83.36) (width 0.2) (layer "B.Cu") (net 12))
 (segment (start 153.9185 116.985314) (end 153.9185 89.2185) (width 0.2) (layer "B.Cu") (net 12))
 (segment (start 150.757814 120.146) (end 153.9185 116.985314) (width 0.2) (layer "B.Cu") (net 12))
 (segment (start 145.451684 122.686) (end 147.991684 120.146) (width 0.2) (layer "B.Cu") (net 12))
 (segment (start 124.7775 121.285) (end 141.846186 121.285) (width 0.2) (layer "B.Cu") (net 12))
 (segment (start 147.991684 120.146) (end 150.757814 120.146) (width 0.2) (layer "B.Cu") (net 12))
 (segment (start 141.846186 121.285) (end 143.247186 122.686) (width 0.2) (layer "B.Cu") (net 12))
 (segment (start 142.4265 84.862) (end 146.72 80.5685) (width 0.2) (layer "F.Cu") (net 3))
 (segment (start 143.8275 121.285) (end 143.8275 104.216314) (width 0.2) (layer "F.Cu") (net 3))
 (segment (start 143.8275 104.216314) (end 142.4265 102.815314) (width 0.2) (layer "F.Cu") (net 3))
 (segment (start 142.4265 102.815314) (end 142.4265 84.862) (width 0.2) (layer "F.Cu") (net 3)))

